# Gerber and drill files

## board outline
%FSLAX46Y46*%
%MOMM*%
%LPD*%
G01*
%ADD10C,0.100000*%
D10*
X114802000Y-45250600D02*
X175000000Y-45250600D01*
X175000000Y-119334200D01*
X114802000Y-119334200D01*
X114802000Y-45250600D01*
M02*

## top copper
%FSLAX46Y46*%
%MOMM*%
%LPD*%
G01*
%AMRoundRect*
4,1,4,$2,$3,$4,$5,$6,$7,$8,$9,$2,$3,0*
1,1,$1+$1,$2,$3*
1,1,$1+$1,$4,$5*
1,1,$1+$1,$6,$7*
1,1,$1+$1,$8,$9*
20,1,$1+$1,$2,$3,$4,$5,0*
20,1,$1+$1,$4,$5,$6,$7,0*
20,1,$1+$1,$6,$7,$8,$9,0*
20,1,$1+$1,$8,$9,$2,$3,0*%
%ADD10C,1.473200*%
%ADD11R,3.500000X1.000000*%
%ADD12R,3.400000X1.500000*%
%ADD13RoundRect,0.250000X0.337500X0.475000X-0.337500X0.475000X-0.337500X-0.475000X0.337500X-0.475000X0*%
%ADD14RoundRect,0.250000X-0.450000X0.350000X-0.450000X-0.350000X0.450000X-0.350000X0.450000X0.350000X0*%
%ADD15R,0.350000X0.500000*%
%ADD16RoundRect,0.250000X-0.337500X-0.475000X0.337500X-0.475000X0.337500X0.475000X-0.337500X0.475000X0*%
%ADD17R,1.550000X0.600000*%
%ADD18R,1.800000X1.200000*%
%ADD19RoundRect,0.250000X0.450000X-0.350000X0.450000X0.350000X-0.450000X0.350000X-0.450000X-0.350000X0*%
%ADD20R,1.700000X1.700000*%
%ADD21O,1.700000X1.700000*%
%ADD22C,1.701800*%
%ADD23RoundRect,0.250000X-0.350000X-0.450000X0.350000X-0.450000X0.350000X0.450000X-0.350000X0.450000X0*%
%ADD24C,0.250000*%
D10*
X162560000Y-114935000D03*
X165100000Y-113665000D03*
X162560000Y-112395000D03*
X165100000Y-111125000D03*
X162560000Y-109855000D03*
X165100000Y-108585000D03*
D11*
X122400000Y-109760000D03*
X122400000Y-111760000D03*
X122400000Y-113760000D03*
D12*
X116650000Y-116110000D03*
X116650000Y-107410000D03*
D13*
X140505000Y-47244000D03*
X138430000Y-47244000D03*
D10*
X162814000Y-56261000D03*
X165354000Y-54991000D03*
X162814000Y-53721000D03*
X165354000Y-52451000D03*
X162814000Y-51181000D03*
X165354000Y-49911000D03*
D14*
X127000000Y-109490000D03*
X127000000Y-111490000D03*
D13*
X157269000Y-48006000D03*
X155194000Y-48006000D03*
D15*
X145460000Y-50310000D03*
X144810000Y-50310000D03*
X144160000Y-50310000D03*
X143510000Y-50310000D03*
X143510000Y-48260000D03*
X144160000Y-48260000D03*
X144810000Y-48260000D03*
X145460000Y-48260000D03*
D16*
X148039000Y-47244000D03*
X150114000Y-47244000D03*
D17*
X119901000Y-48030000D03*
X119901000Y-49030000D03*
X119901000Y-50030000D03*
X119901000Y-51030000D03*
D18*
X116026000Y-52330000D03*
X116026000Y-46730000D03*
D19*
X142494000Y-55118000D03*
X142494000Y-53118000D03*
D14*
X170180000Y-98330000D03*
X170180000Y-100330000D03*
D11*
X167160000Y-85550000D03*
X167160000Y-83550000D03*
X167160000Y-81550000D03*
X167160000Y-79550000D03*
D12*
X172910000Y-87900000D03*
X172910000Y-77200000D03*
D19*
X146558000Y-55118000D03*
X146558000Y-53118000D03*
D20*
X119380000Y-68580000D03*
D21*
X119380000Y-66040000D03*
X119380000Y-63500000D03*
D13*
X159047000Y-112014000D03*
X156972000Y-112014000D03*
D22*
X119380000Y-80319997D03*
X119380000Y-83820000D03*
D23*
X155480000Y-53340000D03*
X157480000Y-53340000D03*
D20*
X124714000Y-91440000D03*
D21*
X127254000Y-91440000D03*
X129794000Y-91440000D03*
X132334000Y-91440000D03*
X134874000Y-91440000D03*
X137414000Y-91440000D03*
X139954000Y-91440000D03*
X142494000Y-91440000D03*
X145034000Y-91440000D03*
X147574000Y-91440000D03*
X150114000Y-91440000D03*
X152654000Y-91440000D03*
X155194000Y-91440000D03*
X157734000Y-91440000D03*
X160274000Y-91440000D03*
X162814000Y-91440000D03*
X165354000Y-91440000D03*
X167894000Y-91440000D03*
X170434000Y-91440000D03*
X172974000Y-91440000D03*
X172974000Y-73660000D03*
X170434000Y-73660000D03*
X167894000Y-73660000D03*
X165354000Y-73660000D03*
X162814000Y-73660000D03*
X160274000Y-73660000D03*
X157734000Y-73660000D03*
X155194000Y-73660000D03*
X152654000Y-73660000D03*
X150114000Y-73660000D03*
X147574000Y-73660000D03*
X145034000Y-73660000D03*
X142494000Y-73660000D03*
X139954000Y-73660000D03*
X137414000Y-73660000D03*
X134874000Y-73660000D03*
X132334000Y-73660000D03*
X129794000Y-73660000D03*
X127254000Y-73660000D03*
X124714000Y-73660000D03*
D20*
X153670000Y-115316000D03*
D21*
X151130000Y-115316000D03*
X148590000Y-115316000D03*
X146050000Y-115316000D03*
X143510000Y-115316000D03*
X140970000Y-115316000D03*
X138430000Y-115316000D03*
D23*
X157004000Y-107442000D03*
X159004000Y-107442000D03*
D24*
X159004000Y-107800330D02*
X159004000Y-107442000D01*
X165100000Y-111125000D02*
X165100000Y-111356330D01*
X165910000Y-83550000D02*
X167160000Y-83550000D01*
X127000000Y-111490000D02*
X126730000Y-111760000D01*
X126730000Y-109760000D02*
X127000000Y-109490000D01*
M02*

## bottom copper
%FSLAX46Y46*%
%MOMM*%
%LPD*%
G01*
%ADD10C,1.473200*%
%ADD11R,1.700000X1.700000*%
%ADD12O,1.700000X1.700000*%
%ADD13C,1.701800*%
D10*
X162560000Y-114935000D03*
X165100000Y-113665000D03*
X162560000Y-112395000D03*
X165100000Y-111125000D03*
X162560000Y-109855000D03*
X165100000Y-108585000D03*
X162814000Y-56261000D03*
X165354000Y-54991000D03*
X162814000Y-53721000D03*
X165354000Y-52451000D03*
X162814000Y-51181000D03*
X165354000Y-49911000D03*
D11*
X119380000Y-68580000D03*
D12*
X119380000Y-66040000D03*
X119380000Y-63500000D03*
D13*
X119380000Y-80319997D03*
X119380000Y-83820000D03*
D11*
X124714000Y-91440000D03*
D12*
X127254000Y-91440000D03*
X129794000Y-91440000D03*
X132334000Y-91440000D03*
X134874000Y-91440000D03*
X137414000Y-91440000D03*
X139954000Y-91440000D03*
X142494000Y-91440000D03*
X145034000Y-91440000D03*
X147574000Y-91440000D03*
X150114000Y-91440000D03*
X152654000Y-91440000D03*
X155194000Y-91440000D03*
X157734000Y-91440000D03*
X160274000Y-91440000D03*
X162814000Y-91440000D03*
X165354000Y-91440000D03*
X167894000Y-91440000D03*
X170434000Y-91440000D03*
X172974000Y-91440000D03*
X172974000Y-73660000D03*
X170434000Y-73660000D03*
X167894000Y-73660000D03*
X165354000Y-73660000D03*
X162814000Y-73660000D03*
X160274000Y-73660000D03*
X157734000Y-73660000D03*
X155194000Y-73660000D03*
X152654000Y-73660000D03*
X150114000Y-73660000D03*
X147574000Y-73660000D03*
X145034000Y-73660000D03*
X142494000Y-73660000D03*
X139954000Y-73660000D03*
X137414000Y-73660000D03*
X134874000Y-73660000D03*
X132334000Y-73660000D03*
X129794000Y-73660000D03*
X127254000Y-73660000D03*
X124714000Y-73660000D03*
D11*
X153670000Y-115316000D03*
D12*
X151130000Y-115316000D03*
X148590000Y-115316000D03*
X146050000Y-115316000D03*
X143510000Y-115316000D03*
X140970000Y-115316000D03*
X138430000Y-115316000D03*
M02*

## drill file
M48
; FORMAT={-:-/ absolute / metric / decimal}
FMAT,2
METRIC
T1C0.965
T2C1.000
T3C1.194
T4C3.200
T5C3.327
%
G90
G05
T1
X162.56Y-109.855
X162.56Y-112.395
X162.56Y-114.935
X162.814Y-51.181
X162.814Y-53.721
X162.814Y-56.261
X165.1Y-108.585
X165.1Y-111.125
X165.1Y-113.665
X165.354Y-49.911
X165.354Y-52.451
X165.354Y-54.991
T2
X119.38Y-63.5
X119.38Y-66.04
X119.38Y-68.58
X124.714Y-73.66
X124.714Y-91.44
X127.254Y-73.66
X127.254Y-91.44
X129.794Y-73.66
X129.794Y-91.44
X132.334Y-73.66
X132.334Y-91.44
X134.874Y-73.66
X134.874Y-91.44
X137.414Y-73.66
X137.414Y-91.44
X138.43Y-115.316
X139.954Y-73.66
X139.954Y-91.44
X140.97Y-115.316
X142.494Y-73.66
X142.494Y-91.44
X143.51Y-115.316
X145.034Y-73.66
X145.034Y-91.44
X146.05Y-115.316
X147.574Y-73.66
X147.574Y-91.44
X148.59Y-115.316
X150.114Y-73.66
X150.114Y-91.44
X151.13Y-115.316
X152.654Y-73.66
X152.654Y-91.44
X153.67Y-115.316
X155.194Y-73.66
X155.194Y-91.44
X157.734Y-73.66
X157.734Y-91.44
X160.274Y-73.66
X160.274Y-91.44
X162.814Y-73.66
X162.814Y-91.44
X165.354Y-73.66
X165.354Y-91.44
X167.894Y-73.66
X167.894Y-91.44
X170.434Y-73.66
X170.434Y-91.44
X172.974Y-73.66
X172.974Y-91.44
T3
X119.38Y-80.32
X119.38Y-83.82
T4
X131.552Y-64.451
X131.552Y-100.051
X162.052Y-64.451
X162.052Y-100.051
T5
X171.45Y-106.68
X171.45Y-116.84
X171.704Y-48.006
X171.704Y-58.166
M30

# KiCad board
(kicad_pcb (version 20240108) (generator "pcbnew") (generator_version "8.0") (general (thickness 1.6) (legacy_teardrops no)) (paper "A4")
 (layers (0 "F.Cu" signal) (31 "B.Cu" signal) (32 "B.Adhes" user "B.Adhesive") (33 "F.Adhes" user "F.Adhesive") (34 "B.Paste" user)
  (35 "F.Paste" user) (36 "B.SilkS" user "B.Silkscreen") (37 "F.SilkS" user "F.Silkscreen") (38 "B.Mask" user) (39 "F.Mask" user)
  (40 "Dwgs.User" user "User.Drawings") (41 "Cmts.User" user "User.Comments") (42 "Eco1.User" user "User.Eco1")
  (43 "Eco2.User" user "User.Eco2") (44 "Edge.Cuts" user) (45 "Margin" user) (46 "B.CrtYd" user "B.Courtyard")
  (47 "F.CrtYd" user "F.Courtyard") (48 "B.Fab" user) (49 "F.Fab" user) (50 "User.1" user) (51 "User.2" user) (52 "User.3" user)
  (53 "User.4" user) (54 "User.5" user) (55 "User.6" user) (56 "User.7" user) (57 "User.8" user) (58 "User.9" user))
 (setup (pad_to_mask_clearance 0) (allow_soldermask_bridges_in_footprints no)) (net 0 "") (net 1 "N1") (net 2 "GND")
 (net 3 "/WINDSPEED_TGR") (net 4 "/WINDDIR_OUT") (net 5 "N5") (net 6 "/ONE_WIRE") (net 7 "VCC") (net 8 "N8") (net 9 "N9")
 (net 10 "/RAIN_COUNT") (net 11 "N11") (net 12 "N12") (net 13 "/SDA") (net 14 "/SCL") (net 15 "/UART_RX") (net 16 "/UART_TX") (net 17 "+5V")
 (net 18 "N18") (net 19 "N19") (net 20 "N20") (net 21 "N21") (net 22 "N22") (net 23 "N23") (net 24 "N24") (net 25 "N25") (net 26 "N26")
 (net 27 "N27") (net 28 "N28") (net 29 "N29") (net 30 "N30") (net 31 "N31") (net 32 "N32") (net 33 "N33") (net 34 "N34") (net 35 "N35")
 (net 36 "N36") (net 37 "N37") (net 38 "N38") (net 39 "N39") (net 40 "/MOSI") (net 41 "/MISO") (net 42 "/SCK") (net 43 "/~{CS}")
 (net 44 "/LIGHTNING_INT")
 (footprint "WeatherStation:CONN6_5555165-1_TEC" (layer "F.Cu") (at 162.56 114.935 90)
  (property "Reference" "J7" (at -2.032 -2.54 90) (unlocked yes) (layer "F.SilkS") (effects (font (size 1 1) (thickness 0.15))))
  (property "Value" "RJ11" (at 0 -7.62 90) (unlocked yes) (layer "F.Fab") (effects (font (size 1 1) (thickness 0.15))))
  (pad "" np_thru_hole circle (at -1.905 8.89 90) (size 3.3274 3.3274) (drill 3.3274) (layers "*.Cu" "*.Mask"))
  (pad "" np_thru_hole circle (at 8.255 8.89 90) (size 3.3274 3.3274) (drill 3.3274) (layers "*.Cu" "*.Mask"))
  (pad "1" thru_hole circle (at 0 0 90) (size 1.4732 1.4732) (drill 0.9652) (layers "*.Cu" "*.Mask") (remove_unused_layers no) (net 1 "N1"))
  (pad "2" thru_hole circle (at 1.27 2.54 90) (size 1.4732 1.4732) (drill 0.9652) (layers "*.Cu" "*.Mask") (remove_unused_layers no)
   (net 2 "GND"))
  (pad "3" thru_hole circle (at 2.54 0 90) (size 1.4732 1.4732) (drill 0.9652) (layers "*.Cu" "*.Mask") (remove_unused_layers no)
   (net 2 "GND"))
  (pad "4" thru_hole circle (at 3.81 2.54 90) (size 1.4732 1.4732) (drill 0.9652) (layers "*.Cu" "*.Mask") (remove_unused_layers no)
   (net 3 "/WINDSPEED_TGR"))
  (pad "5" thru_hole circle (at 5.08 0 90) (size 1.4732 1.4732) (drill 0.9652) (layers "*.Cu" "*.Mask") (remove_unused_layers no)
   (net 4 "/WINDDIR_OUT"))
  (pad "6" thru_hole circle (at 6.35 2.54 90) (size 1.4732 1.4732) (drill 0.9652) (layers "*.Cu" "*.Mask") (remove_unused_layers no)
   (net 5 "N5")))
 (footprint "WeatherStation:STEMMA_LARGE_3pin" (layer "F.Cu") (at 120.65 111.76 -90)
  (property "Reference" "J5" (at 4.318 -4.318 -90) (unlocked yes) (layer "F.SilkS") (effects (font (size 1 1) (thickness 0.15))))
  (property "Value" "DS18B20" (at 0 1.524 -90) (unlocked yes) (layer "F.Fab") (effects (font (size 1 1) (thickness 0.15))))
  (pad "1" smd rect (at -2 -1.75 270) (size 1 3.5) (layers "F.Cu" "F.Paste" "F.Mask") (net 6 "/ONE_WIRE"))
  (pad "2" smd rect (at 0 -1.75 270) (size 1 3.5) (layers "F.Cu" "F.Paste" "F.Mask") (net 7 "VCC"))
  (pad "3" smd rect (at 2 -1.75 270) (size 1 3.5) (layers "F.Cu" "F.Paste" "F.Mask") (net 2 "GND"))
  (pad "4" smd rect (at 4.35 4 270) (size 1.5 3.4) (layers "F.Cu" "F.Paste" "F.Mask"))
  (pad "5" smd rect (at -4.35 4 270) (size 1.5 3.4) (layers "F.Cu" "F.Paste" "F.Mask")))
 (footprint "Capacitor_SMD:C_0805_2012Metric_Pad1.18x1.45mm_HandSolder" (layer "F.Cu") (at 139.4675 47.244 180)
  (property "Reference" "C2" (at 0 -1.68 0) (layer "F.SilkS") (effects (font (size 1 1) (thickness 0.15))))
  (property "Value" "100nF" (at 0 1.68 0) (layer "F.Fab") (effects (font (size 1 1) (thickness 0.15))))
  (pad "1" smd roundrect (at -1.0375 0 180) (size 1.175 1.45) (layers "F.Cu" "F.Paste" "F.Mask") (roundrect_rratio 0.212766) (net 7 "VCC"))
  (pad "2" smd roundrect (at 1.0375 0 180) (size 1.175 1.45) (layers "F.Cu" "F.Paste" "F.Mask") (roundrect_rratio 0.212766) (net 2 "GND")))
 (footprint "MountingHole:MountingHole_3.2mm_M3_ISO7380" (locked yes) (layer "F.Cu") (at 162.052 64.4506)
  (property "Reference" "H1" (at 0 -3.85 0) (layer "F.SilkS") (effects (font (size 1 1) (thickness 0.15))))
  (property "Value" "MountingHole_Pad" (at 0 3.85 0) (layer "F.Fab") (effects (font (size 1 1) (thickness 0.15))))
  (pad "" np_thru_hole circle (at 0 0) (size 3.2 3.2) (drill 3.2) (layers "*.Cu" "*.Mask")))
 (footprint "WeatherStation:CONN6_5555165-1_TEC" (layer "F.Cu") (at 162.814 56.261 90)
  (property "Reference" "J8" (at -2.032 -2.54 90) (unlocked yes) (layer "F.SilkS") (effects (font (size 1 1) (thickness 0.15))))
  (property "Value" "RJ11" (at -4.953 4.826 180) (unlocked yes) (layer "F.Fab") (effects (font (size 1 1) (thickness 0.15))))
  (pad "" np_thru_hole circle (at -1.905 8.89 90) (size 3.3274 3.3274) (drill 3.3274) (layers "*.Cu" "*.Mask"))
  (pad "" np_thru_hole circle (at 8.255 8.89 90) (size 3.3274 3.3274) (drill 3.3274) (layers "F&B.Cu" "*.Mask"))
  (pad "1" thru_hole circle (at 0 0 90) (size 1.4732 1.4732) (drill 0.9652) (layers "*.Cu" "*.Mask") (remove_unused_layers no) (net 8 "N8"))
  (pad "2" thru_hole circle (at 1.27 2.54 90) (size 1.4732 1.4732) (drill 0.9652) (layers "*.Cu" "*.Mask") (remove_unused_layers no)
   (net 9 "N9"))
  (pad "3" thru_hole circle (at 2.54 0 90) (size 1.4732 1.4732) (drill 0.9652) (layers "*.Cu" "*.Mask") (remove_unused_layers no)
   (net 2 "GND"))
  (pad "4" thru_hole circle (at 3.81 2.54 90) (size 1.4732 1.4732) (drill 0.9652) (layers "*.Cu" "*.Mask") (remove_unused_layers no)
   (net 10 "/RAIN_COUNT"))
  (pad "5" thru_hole circle (at 5.08 0 90) (size 1.4732 1.4732) (drill 0.9652) (layers "*.Cu" "*.Mask") (remove_unused_layers no)
   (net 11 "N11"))
  (pad "6" thru_hole circle (at 6.35 2.54 90) (size 1.4732 1.4732) (drill 0.9652) (layers "*.Cu" "*.Mask") (remove_unused_layers no)
   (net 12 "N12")))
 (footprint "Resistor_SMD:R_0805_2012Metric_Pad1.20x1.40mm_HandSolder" (layer "F.Cu") (at 127 110.49 -90)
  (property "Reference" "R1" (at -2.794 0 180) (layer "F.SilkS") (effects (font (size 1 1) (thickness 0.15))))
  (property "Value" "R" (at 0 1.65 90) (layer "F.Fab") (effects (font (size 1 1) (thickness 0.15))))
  (pad "1" smd roundrect (at -1 0 270) (size 1.2 1.4) (layers "F.Cu" "F.Paste" "F.Mask") (roundrect_rratio 0.208333) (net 6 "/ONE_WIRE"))
  (pad "2" smd roundrect (at 1 0 270) (size 1.2 1.4) (layers "F.Cu" "F.Paste" "F.Mask") (roundrect_rratio 0.208333) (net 7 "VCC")))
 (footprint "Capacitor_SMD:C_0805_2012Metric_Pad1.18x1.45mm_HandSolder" (layer "F.Cu") (at 156.2315 48.006 180)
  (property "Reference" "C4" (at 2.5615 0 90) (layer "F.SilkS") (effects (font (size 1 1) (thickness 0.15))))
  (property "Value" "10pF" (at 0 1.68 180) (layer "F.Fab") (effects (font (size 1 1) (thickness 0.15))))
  (pad "1" smd roundrect (at -1.0375 0 180) (size 1.175 1.45) (layers "F.Cu" "F.Paste" "F.Mask") (roundrect_rratio 0.212766)
   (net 10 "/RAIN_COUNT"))
  (pad "2" smd roundrect (at 1.0375 0 180) (size 1.175 1.45) (layers "F.Cu" "F.Paste" "F.Mask") (roundrect_rratio 0.212766) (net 2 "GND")))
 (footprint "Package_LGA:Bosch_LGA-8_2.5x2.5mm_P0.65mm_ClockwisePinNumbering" (layer "F.Cu") (at 144.485 49.285 180)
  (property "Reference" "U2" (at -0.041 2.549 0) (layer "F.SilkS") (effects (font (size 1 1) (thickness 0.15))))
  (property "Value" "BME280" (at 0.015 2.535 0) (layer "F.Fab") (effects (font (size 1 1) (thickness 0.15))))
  (pad "1" smd rect (at -0.975 -1.025 270) (size 0.5 0.35) (layers "F.Cu" "F.Paste" "F.Mask") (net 2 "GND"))
  (pad "2" smd rect (at -0.325 -1.025 270) (size 0.5 0.35) (layers "F.Cu" "F.Paste" "F.Mask") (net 7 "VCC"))
  (pad "3" smd rect (at 0.325 -1.025 270) (size 0.5 0.35) (layers "F.Cu" "F.Paste" "F.Mask") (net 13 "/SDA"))
  (pad "4" smd rect (at 0.975 -1.025 270) (size 0.5 0.35) (layers "F.Cu" "F.Paste" "F.Mask") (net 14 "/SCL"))
  (pad "5" smd rect (at 0.975 1.025 270) (size 0.5 0.35) (layers "F.Cu" "F.Paste" "F.Mask") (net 2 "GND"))
  (pad "6" smd rect (at 0.325 1.025 270) (size 0.5 0.35) (layers "F.Cu" "F.Paste" "F.Mask") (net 7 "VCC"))
  (pad "7" smd rect (at -0.325 1.025 270) (size 0.5 0.35) (layers "F.Cu" "F.Paste" "F.Mask") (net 2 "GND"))
  (pad "8" smd rect (at -0.975 1.025 270) (size 0.5 0.35) (layers "F.Cu" "F.Paste" "F.Mask") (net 7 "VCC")))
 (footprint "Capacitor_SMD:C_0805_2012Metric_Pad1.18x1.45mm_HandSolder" (layer "F.Cu") (at 149.0765 47.244)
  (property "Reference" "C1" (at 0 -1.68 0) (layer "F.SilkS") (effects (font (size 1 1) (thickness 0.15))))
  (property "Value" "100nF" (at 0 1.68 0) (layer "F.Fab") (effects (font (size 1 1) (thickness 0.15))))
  (pad "1" smd roundrect (at -1.0375 0) (size 1.175 1.45) (layers "F.Cu" "F.Paste" "F.Mask") (roundrect_rratio 0.212766) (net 7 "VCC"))
  (pad "2" smd roundrect (at 1.0375 0) (size 1.175 1.45) (layers "F.Cu" "F.Paste" "F.Mask") (roundrect_rratio 0.212766) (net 2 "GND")))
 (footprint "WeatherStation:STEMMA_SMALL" (layer "F.Cu") (at 119.126 49.53 -90)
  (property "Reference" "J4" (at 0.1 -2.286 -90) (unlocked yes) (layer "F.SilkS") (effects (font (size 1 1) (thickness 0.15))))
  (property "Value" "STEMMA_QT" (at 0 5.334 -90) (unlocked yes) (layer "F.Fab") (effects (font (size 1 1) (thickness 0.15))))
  (pad "1" smd rect (at -1.5 -0.775 270) (size 0.6 1.55) (layers "F.Cu" "F.Paste" "F.Mask") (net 2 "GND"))
  (pad "2" smd rect (at -0.5 -0.775 270) (size 0.6 1.55) (layers "F.Cu" "F.Paste" "F.Mask") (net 7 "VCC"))
  (pad "3" smd rect (at 0.5 -0.775 270) (size 0.6 1.55) (layers "F.Cu" "F.Paste" "F.Mask") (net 13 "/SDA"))
  (pad "4" smd rect (at 1.5 -0.775 270) (size 0.6 1.55) (layers "F.Cu" "F.Paste" "F.Mask") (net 14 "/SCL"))
  (pad "5" smd rect (at 2.8 3.1 270) (size 1.2 1.8) (layers "F.Cu" "F.Paste" "F.Mask"))
  (pad "6" smd rect (at -2.8 3.1 270) (size 1.2 1.8) (layers "F.Cu" "F.Paste" "F.Mask")))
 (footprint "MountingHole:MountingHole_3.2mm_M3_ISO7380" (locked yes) (layer "F.Cu") (at 162.052 100.0506)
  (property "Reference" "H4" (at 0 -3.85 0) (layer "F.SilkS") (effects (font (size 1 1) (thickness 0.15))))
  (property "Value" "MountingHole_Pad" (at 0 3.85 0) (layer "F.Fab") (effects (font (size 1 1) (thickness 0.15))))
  (pad "" np_thru_hole circle (at 0 0) (size 3.2 3.2) (drill 3.2) (layers "*.Cu" "*.Mask")))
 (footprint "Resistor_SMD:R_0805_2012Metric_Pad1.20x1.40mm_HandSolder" (layer "F.Cu") (at 142.494 54.118 90)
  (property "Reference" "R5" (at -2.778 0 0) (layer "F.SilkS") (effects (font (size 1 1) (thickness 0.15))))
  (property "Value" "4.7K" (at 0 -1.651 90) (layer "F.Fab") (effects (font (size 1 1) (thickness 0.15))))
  (pad "1" smd roundrect (at -1 0 90) (size 1.2 1.4) (layers "F.Cu" "F.Paste" "F.Mask") (roundrect_rratio 0.208333) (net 7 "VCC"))
  (pad "2" smd roundrect (at 1 0 90) (size 1.2 1.4) (layers "F.Cu" "F.Paste" "F.Mask") (roundrect_rratio 0.208333) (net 14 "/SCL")))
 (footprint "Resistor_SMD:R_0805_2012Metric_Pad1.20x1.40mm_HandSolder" (layer "F.Cu") (at 170.18 99.33 -90)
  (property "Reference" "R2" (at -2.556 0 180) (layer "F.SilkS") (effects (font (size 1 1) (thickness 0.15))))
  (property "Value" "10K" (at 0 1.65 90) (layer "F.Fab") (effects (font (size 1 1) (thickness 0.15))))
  (pad "1" smd roundrect (at -1 0 270) (size 1.2 1.4) (layers "F.Cu" "F.Paste" "F.Mask") (roundrect_rratio 0.208333) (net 7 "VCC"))
  (pad "2" smd roundrect (at 1 0 270) (size 1.2 1.4) (layers "F.Cu" "F.Paste" "F.Mask") (roundrect_rratio 0.208333) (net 4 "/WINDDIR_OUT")))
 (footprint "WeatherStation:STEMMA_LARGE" (layer "F.Cu") (at 168.91 82.55 90)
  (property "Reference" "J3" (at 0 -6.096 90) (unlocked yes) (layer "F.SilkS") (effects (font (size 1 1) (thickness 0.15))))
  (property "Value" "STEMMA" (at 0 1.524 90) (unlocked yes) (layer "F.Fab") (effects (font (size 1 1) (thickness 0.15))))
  (pad "1" smd rect (at -3 -1.75 90) (size 1 3.5) (layers "F.Cu" "F.Paste" "F.Mask") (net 2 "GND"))
  (pad "2" smd rect (at -1 -1.75 90) (size 1 3.5) (layers "F.Cu" "F.Paste" "F.Mask") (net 7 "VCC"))
  (pad "3" smd rect (at 1 -1.75 90) (size 1 3.5) (layers "F.Cu" "F.Paste" "F.Mask") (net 13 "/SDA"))
  (pad "4" smd rect (at 3 -1.75 90) (size 1 3.5) (layers "F.Cu" "F.Paste" "F.Mask") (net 14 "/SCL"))
  (pad "5" smd rect (at -5.35 4 90) (size 1.5 3.4) (layers "F.Cu" "F.Paste" "F.Mask"))
  (pad "6" smd rect (at 5.35 4 90) (size 1.5 3.4) (layers "F.Cu" "F.Paste" "F.Mask")))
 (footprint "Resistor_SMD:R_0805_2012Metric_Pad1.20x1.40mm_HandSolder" (layer "F.Cu") (at 146.558 54.118 90)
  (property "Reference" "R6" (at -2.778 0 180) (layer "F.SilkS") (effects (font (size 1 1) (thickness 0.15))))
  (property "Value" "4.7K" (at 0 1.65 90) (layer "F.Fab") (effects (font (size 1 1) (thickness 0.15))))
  (pad "1" smd roundrect (at -1 0 90) (size 1.2 1.4) (layers "F.Cu" "F.Paste" "F.Mask") (roundrect_rratio 0.208333) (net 7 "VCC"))
  (pad "2" smd roundrect (at 1 0 90) (size 1.2 1.4) (layers "F.Cu" "F.Paste" "F.Mask") (roundrect_rratio 0.208333) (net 13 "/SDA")))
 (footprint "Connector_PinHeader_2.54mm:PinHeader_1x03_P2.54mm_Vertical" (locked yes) (layer "F.Cu") (at 119.38 68.58 180)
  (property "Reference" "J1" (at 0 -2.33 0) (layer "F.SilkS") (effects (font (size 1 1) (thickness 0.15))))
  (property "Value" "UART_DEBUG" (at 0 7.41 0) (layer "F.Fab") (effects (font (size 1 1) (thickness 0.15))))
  (pad "1" thru_hole rect (at 0 0 180) (size 1.7 1.7) (drill 1) (layers "*.Cu" "*.Mask") (remove_unused_layers no) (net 2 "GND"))
  (pad "2" thru_hole oval (at 0 2.54 180) (size 1.7 1.7) (drill 1) (layers "*.Cu" "*.Mask") (remove_unused_layers no) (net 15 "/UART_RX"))
  (pad "3" thru_hole oval (at 0 5.08 180) (size 1.7 1.7) (drill 1) (layers "*.Cu" "*.Mask") (remove_unused_layers no) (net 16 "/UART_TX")))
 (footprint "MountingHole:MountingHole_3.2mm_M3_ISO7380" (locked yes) (layer "F.Cu") (at 131.552 100.0506)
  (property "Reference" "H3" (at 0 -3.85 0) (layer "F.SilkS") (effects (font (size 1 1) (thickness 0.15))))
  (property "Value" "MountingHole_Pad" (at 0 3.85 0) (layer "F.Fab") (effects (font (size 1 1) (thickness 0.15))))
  (pad "" np_thru_hole circle (at 0 0) (size 3.2 3.2) (drill 3.2) (layers "*.Cu" "*.Mask")))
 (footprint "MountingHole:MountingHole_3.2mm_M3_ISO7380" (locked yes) (layer "F.Cu") (at 131.552 64.4506)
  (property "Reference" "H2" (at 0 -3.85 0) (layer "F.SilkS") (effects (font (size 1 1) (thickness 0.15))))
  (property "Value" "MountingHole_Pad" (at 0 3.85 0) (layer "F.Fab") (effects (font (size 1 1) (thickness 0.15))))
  (pad "" np_thru_hole circle (at 0 0) (size 3.2 3.2) (drill 3.2) (layers "*.Cu" "*.Mask")))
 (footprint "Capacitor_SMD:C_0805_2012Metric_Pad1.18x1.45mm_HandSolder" (layer "F.Cu") (at 158.0095 112.014 180)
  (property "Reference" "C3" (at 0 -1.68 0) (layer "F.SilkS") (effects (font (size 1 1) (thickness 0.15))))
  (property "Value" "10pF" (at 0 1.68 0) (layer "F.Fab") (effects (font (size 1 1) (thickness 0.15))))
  (pad "1" smd roundrect (at -1.0375 0 180) (size 1.175 1.45) (layers "F.Cu" "F.Paste" "F.Mask") (roundrect_rratio 0.212766)
   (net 3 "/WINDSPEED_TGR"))
  (pad "2" smd roundrect (at 1.0375 0 180) (size 1.175 1.45) (layers "F.Cu" "F.Paste" "F.Mask") (roundrect_rratio 0.212766) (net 2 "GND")))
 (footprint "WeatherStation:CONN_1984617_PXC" (layer "F.Cu") (at 119.38 80.319998 -90)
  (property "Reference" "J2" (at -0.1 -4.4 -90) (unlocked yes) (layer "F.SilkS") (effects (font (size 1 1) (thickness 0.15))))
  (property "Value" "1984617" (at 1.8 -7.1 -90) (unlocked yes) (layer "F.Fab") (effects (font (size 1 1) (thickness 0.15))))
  (pad "1" thru_hole circle (at -0.000001 0 270) (size 1.7018 1.7018) (drill 1.1938) (layers "*.Cu" "*.Mask") (remove_unused_layers no)
   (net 2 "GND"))
  (pad "2" thru_hole circle (at 3.500002 0 270) (size 1.7018 1.7018) (drill 1.1938) (layers "*.Cu" "*.Mask") (remove_unused_layers no)
   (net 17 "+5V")))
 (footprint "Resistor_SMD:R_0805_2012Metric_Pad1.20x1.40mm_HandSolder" (layer "F.Cu") (at 156.48 53.34)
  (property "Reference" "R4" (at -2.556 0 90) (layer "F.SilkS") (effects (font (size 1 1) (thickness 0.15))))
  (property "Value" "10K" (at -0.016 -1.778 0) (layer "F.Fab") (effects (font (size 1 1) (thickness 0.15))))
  (pad "1" smd roundrect (at -1 0) (size 1.2 1.4) (layers "F.Cu" "F.Paste" "F.Mask") (roundrect_rratio 0.208333) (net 7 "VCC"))
  (pad "2" smd roundrect (at 1 0) (size 1.2 1.4) (layers "F.Cu" "F.Paste" "F.Mask") (roundrect_rratio 0.208333) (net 10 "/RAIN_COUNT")))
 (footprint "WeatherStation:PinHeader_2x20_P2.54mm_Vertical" (layer "F.Cu") (at 124.714 82.55 90)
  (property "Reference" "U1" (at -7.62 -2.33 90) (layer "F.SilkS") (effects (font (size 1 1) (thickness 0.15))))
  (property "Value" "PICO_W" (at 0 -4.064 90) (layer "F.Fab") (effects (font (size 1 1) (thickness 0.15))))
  (pad "1" thru_hole rect (at -8.89 0 90) (size 1.7 1.7) (drill 1) (layers "*.Cu" "*.Mask") (remove_unused_layers no) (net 16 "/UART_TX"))
  (pad "2" thru_hole oval (at -8.89 2.54 90) (size 1.7 1.7) (drill 1) (layers "*.Cu" "*.Mask") (remove_unused_layers no) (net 15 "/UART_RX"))
  (pad "3" thru_hole oval (at -8.89 5.08 90) (size 1.7 1.7) (drill 1) (layers "*.Cu" "*.Mask") (remove_unused_layers no) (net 2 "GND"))
  (pad "4" thru_hole oval (at -8.89 7.62 90) (size 1.7 1.7) (drill 1) (layers "*.Cu" "*.Mask") (remove_unused_layers no) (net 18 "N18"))
  (pad "5" thru_hole oval (at -8.89 10.16 90) (size 1.7 1.7) (drill 1) (layers "*.Cu" "*.Mask") (remove_unused_layers no) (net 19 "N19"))
  (pad "6" thru_hole oval (at -8.89 12.7 90) (size 1.7 1.7) (drill 1) (layers "*.Cu" "*.Mask") (remove_unused_layers no)
   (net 10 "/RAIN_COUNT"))
  (pad "7" thru_hole oval (at -8.89 15.24 90) (size 1.7 1.7) (drill 1) (layers "*.Cu" "*.Mask") (remove_unused_layers no) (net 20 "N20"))
  (pad "8" thru_hole oval (at -8.89 17.78 90) (size 1.7 1.7) (drill 1) (layers "*.Cu" "*.Mask") (remove_unused_layers no) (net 2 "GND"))
  (pad "9" thru_hole oval (at -8.89 20.32 90) (size 1.7 1.7) (drill 1) (layers "*.Cu" "*.Mask") (remove_unused_layers no) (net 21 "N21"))
  (pad "10" thru_hole oval (at -8.89 22.86 90) (size 1.7 1.7) (drill 1) (layers "*.Cu" "*.Mask") (remove_unused_layers no) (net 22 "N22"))
  (pad "11" thru_hole oval (at -8.89 25.4 90) (size 1.7 1.7) (drill 1) (layers "*.Cu" "*.Mask") (remove_unused_layers no) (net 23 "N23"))
  (pad "12" thru_hole oval (at -8.89 27.94 90) (size 1.7 1.7) (drill 1) (layers "*.Cu" "*.Mask") (remove_unused_layers no) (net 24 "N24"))
  (pad "13" thru_hole oval (at -8.89 30.48 90) (size 1.7 1.7) (drill 1) (layers "*.Cu" "*.Mask") (remove_unused_layers no) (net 2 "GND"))
  (pad "14" thru_hole oval (at -8.89 33.02 90) (size 1.7 1.7) (drill 1) (layers "*.Cu" "*.Mask") (remove_unused_layers no) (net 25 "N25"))
  (pad "15" thru_hole oval (at -8.89 35.56 90) (size 1.7 1.7) (drill 1) (layers "*.Cu" "*.Mask") (remove_unused_layers no) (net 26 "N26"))
  (pad "16" thru_hole oval (at -8.89 38.1 90) (size 1.7 1.7) (drill 1) (layers "*.Cu" "*.Mask") (remove_unused_layers no) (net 13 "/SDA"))
  (pad "17" thru_hole oval (at -8.89 40.64 90) (size 1.7 1.7) (drill 1) (layers "*.Cu" "*.Mask") (remove_unused_layers no) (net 14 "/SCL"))
  (pad "18" thru_hole oval (at -8.89 43.18 90) (size 1.7 1.7) (drill 1) (layers "*.Cu" "*.Mask") (remove_unused_layers no) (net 2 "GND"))
  (pad "19" thru_hole oval (at -8.89 45.72 90) (size 1.7 1.7) (drill 1) (layers "*.Cu" "*.Mask") (remove_unused_layers no) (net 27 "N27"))
  (pad "20" thru_hole oval (at -8.89 48.26 90) (size 1.7 1.7) (drill 1) (layers "*.Cu" "*.Mask") (remove_unused_layers no)
   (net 6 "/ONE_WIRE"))
  (pad "21" thru_hole oval (at 8.89 48.26 90) (size 1.7 1.7) (drill 1) (layers "*.Cu" "*.Mask") (remove_unused_layers no) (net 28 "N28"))
  (pad "22" thru_hole oval (at 8.89 45.72 90) (size 1.7 1.7) (drill 1) (layers "*.Cu" "*.Mask") (remove_unused_layers no) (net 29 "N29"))
  (pad "23" thru_hole oval (at 8.89 43.18 90) (size 1.7 1.7) (drill 1) (layers "*.Cu" "*.Mask") (remove_unused_layers no) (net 2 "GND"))
  (pad "24" thru_hole oval (at 8.89 40.64 90) (size 1.7 1.7) (drill 1) (layers "*.Cu" "*.Mask") (remove_unused_layers no) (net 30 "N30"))
  (pad "25" thru_hole oval (at 8.89 38.1 90) (size 1.7 1.7) (drill 1) (layers "*.Cu" "*.Mask") (remove_unused_layers no) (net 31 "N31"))
  (pad "26" thru_hole oval (at 8.89 35.56 90) (size 1.7 1.7) (drill 1) (layers "*.Cu" "*.Mask") (remove_unused_layers no) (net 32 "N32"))
  (pad "27" thru_hole oval (at 8.89 33.02 90) (size 1.7 1.7) (drill 1) (layers "*.Cu" "*.Mask") (remove_unused_layers no) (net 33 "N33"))
  (pad "28" thru_hole oval (at 8.89 30.48 90) (size 1.7 1.7) (drill 1) (layers "*.Cu" "*.Mask") (remove_unused_layers no) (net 2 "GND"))
  (pad "29" thru_hole oval (at 8.89 27.94 90) (size 1.7 1.7) (drill 1) (layers "*.Cu" "*.Mask") (remove_unused_layers no)
   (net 3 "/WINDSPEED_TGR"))
  (pad "30" thru_hole oval (at 8.89 25.4 90) (size 1.7 1.7) (drill 1) (layers "*.Cu" "*.Mask") (remove_unused_layers no) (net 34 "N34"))
  (pad "31" thru_hole oval (at 8.89 22.86 90) (size 1.7 1.7) (drill 1) (layers "*.Cu" "*.Mask") (remove_unused_layers no)
   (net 4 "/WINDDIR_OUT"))
  (pad "32" thru_hole oval (at 8.89 20.32 90) (size 1.7 1.7) (drill 1) (layers "*.Cu" "*.Mask") (remove_unused_layers no) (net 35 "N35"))
  (pad "33" thru_hole oval (at 8.89 17.78 90) (size 1.7 1.7) (drill 1) (layers "*.Cu" "*.Mask") (remove_unused_layers no) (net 2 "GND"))
  (pad "34" thru_hole oval (at 8.89 15.24 90) (size 1.7 1.7) (drill 1) (layers "*.Cu" "*.Mask") (remove_unused_layers no) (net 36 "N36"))
  (pad "35" thru_hole oval (at 8.89 12.7 90) (size 1.7 1.7) (drill 1) (layers "*.Cu" "*.Mask") (remove_unused_layers no) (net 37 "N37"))
  (pad "36" thru_hole oval (at 8.89 10.16 90) (size 1.7 1.7) (drill 1) (layers "*.Cu" "*.Mask") (remove_unused_layers no) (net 7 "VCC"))
  (pad "37" thru_hole oval (at 8.89 7.62 90) (size 1.7 1.7) (drill 1) (layers "*.Cu" "*.Mask") (remove_unused_layers no) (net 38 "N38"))
  (pad "38" thru_hole oval (at 8.89 5.08 90) (size 1.7 1.7) (drill 1) (layers "*.Cu" "*.Mask") (remove_unused_layers no) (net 2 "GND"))
  (pad "39" thru_hole oval (at 8.89 2.54 90) (size 1.7 1.7) (drill 1) (layers "*.Cu" "*.Mask") (remove_unused_layers no) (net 17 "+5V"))
  (pad "40" thru_hole oval (at 8.89 0 90) (size 1.7 1.7) (drill 1) (layers "*.Cu" "*.Mask") (remove_unused_layers no) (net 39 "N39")))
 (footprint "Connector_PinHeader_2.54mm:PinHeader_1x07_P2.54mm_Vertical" (layer "F.Cu") (at 153.67 115.316 -90)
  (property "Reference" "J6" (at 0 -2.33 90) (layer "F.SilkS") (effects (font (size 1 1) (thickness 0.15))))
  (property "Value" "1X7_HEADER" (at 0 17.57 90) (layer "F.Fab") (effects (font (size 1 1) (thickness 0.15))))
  (pad "1" thru_hole rect (at 0 0 270) (size 1.7 1.7) (drill 1) (layers "*.Cu" "*.Mask") (remove_unused_layers no) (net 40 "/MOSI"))
  (pad "2" thru_hole oval (at 0 2.54 270) (size 1.7 1.7) (drill 1) (layers "*.Cu" "*.Mask") (remove_unused_layers no) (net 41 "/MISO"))
  (pad "3" thru_hole oval (at 0 5.08 270) (size 1.7 1.7) (drill 1) (layers "*.Cu" "*.Mask") (remove_unused_layers no) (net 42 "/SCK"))
  (pad "4" thru_hole oval (at 0 7.62 270) (size 1.7 1.7) (drill 1) (layers "*.Cu" "*.Mask") (remove_unused_layers no) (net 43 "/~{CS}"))
  (pad "5" thru_hole oval (at 0 10.16 270) (size 1.7 1.7) (drill 1) (layers "*.Cu" "*.Mask") (remove_unused_layers no)
   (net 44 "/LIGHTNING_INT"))
  (pad "6" thru_hole oval (at 0 12.7 270) (size 1.7 1.7) (drill 1) (layers "*.Cu" "*.Mask") (remove_unused_layers no) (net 7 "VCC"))
  (pad "7" thru_hole oval (at 0 15.24 270) (size 1.7 1.7) (drill 1) (layers "*.Cu" "*.Mask") (remove_unused_layers no) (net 2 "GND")))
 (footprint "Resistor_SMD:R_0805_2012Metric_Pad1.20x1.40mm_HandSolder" (layer "F.Cu") (at 158.004 107.442)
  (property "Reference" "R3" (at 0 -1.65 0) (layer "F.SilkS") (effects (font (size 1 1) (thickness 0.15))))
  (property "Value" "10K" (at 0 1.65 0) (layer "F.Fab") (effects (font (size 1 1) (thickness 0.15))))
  (pad "1" smd roundrect (at -1 0) (size 1.2 1.4) (layers "F.Cu" "F.Paste" "F.Mask") (roundrect_rratio 0.208333) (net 7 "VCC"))
  (pad "2" smd roundrect (at 1 0) (size 1.2 1.4) (layers "F.Cu" "F.Paste" "F.Mask") (roundrect_rratio 0.208333) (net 3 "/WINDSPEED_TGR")))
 (gr_rect (start 114.802 45.2506) (end 175 119.3342) (stroke (width 0.1) (type default)) (fill none) (layer "Edge.Cuts"))
 (segment (start 159.004 107.80033) (end 159.004 107.442) (width 0.25) (layer "F.Cu") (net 3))
 (segment (start 165.1 111.125) (end 165.1 111.35633) (width 0.25) (layer "F.Cu") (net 3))
 (segment (start 165.91 83.55) (end 167.16 83.55) (width 0.25) (layer "F.Cu") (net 7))
 (segment (start 127 111.49) (end 126.73 111.76) (width 0.25) (layer "F.Cu") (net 7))
 (segment (start 126.73 109.76) (end 127 109.49) (width 0.25) (layer "F.Cu") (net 6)))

